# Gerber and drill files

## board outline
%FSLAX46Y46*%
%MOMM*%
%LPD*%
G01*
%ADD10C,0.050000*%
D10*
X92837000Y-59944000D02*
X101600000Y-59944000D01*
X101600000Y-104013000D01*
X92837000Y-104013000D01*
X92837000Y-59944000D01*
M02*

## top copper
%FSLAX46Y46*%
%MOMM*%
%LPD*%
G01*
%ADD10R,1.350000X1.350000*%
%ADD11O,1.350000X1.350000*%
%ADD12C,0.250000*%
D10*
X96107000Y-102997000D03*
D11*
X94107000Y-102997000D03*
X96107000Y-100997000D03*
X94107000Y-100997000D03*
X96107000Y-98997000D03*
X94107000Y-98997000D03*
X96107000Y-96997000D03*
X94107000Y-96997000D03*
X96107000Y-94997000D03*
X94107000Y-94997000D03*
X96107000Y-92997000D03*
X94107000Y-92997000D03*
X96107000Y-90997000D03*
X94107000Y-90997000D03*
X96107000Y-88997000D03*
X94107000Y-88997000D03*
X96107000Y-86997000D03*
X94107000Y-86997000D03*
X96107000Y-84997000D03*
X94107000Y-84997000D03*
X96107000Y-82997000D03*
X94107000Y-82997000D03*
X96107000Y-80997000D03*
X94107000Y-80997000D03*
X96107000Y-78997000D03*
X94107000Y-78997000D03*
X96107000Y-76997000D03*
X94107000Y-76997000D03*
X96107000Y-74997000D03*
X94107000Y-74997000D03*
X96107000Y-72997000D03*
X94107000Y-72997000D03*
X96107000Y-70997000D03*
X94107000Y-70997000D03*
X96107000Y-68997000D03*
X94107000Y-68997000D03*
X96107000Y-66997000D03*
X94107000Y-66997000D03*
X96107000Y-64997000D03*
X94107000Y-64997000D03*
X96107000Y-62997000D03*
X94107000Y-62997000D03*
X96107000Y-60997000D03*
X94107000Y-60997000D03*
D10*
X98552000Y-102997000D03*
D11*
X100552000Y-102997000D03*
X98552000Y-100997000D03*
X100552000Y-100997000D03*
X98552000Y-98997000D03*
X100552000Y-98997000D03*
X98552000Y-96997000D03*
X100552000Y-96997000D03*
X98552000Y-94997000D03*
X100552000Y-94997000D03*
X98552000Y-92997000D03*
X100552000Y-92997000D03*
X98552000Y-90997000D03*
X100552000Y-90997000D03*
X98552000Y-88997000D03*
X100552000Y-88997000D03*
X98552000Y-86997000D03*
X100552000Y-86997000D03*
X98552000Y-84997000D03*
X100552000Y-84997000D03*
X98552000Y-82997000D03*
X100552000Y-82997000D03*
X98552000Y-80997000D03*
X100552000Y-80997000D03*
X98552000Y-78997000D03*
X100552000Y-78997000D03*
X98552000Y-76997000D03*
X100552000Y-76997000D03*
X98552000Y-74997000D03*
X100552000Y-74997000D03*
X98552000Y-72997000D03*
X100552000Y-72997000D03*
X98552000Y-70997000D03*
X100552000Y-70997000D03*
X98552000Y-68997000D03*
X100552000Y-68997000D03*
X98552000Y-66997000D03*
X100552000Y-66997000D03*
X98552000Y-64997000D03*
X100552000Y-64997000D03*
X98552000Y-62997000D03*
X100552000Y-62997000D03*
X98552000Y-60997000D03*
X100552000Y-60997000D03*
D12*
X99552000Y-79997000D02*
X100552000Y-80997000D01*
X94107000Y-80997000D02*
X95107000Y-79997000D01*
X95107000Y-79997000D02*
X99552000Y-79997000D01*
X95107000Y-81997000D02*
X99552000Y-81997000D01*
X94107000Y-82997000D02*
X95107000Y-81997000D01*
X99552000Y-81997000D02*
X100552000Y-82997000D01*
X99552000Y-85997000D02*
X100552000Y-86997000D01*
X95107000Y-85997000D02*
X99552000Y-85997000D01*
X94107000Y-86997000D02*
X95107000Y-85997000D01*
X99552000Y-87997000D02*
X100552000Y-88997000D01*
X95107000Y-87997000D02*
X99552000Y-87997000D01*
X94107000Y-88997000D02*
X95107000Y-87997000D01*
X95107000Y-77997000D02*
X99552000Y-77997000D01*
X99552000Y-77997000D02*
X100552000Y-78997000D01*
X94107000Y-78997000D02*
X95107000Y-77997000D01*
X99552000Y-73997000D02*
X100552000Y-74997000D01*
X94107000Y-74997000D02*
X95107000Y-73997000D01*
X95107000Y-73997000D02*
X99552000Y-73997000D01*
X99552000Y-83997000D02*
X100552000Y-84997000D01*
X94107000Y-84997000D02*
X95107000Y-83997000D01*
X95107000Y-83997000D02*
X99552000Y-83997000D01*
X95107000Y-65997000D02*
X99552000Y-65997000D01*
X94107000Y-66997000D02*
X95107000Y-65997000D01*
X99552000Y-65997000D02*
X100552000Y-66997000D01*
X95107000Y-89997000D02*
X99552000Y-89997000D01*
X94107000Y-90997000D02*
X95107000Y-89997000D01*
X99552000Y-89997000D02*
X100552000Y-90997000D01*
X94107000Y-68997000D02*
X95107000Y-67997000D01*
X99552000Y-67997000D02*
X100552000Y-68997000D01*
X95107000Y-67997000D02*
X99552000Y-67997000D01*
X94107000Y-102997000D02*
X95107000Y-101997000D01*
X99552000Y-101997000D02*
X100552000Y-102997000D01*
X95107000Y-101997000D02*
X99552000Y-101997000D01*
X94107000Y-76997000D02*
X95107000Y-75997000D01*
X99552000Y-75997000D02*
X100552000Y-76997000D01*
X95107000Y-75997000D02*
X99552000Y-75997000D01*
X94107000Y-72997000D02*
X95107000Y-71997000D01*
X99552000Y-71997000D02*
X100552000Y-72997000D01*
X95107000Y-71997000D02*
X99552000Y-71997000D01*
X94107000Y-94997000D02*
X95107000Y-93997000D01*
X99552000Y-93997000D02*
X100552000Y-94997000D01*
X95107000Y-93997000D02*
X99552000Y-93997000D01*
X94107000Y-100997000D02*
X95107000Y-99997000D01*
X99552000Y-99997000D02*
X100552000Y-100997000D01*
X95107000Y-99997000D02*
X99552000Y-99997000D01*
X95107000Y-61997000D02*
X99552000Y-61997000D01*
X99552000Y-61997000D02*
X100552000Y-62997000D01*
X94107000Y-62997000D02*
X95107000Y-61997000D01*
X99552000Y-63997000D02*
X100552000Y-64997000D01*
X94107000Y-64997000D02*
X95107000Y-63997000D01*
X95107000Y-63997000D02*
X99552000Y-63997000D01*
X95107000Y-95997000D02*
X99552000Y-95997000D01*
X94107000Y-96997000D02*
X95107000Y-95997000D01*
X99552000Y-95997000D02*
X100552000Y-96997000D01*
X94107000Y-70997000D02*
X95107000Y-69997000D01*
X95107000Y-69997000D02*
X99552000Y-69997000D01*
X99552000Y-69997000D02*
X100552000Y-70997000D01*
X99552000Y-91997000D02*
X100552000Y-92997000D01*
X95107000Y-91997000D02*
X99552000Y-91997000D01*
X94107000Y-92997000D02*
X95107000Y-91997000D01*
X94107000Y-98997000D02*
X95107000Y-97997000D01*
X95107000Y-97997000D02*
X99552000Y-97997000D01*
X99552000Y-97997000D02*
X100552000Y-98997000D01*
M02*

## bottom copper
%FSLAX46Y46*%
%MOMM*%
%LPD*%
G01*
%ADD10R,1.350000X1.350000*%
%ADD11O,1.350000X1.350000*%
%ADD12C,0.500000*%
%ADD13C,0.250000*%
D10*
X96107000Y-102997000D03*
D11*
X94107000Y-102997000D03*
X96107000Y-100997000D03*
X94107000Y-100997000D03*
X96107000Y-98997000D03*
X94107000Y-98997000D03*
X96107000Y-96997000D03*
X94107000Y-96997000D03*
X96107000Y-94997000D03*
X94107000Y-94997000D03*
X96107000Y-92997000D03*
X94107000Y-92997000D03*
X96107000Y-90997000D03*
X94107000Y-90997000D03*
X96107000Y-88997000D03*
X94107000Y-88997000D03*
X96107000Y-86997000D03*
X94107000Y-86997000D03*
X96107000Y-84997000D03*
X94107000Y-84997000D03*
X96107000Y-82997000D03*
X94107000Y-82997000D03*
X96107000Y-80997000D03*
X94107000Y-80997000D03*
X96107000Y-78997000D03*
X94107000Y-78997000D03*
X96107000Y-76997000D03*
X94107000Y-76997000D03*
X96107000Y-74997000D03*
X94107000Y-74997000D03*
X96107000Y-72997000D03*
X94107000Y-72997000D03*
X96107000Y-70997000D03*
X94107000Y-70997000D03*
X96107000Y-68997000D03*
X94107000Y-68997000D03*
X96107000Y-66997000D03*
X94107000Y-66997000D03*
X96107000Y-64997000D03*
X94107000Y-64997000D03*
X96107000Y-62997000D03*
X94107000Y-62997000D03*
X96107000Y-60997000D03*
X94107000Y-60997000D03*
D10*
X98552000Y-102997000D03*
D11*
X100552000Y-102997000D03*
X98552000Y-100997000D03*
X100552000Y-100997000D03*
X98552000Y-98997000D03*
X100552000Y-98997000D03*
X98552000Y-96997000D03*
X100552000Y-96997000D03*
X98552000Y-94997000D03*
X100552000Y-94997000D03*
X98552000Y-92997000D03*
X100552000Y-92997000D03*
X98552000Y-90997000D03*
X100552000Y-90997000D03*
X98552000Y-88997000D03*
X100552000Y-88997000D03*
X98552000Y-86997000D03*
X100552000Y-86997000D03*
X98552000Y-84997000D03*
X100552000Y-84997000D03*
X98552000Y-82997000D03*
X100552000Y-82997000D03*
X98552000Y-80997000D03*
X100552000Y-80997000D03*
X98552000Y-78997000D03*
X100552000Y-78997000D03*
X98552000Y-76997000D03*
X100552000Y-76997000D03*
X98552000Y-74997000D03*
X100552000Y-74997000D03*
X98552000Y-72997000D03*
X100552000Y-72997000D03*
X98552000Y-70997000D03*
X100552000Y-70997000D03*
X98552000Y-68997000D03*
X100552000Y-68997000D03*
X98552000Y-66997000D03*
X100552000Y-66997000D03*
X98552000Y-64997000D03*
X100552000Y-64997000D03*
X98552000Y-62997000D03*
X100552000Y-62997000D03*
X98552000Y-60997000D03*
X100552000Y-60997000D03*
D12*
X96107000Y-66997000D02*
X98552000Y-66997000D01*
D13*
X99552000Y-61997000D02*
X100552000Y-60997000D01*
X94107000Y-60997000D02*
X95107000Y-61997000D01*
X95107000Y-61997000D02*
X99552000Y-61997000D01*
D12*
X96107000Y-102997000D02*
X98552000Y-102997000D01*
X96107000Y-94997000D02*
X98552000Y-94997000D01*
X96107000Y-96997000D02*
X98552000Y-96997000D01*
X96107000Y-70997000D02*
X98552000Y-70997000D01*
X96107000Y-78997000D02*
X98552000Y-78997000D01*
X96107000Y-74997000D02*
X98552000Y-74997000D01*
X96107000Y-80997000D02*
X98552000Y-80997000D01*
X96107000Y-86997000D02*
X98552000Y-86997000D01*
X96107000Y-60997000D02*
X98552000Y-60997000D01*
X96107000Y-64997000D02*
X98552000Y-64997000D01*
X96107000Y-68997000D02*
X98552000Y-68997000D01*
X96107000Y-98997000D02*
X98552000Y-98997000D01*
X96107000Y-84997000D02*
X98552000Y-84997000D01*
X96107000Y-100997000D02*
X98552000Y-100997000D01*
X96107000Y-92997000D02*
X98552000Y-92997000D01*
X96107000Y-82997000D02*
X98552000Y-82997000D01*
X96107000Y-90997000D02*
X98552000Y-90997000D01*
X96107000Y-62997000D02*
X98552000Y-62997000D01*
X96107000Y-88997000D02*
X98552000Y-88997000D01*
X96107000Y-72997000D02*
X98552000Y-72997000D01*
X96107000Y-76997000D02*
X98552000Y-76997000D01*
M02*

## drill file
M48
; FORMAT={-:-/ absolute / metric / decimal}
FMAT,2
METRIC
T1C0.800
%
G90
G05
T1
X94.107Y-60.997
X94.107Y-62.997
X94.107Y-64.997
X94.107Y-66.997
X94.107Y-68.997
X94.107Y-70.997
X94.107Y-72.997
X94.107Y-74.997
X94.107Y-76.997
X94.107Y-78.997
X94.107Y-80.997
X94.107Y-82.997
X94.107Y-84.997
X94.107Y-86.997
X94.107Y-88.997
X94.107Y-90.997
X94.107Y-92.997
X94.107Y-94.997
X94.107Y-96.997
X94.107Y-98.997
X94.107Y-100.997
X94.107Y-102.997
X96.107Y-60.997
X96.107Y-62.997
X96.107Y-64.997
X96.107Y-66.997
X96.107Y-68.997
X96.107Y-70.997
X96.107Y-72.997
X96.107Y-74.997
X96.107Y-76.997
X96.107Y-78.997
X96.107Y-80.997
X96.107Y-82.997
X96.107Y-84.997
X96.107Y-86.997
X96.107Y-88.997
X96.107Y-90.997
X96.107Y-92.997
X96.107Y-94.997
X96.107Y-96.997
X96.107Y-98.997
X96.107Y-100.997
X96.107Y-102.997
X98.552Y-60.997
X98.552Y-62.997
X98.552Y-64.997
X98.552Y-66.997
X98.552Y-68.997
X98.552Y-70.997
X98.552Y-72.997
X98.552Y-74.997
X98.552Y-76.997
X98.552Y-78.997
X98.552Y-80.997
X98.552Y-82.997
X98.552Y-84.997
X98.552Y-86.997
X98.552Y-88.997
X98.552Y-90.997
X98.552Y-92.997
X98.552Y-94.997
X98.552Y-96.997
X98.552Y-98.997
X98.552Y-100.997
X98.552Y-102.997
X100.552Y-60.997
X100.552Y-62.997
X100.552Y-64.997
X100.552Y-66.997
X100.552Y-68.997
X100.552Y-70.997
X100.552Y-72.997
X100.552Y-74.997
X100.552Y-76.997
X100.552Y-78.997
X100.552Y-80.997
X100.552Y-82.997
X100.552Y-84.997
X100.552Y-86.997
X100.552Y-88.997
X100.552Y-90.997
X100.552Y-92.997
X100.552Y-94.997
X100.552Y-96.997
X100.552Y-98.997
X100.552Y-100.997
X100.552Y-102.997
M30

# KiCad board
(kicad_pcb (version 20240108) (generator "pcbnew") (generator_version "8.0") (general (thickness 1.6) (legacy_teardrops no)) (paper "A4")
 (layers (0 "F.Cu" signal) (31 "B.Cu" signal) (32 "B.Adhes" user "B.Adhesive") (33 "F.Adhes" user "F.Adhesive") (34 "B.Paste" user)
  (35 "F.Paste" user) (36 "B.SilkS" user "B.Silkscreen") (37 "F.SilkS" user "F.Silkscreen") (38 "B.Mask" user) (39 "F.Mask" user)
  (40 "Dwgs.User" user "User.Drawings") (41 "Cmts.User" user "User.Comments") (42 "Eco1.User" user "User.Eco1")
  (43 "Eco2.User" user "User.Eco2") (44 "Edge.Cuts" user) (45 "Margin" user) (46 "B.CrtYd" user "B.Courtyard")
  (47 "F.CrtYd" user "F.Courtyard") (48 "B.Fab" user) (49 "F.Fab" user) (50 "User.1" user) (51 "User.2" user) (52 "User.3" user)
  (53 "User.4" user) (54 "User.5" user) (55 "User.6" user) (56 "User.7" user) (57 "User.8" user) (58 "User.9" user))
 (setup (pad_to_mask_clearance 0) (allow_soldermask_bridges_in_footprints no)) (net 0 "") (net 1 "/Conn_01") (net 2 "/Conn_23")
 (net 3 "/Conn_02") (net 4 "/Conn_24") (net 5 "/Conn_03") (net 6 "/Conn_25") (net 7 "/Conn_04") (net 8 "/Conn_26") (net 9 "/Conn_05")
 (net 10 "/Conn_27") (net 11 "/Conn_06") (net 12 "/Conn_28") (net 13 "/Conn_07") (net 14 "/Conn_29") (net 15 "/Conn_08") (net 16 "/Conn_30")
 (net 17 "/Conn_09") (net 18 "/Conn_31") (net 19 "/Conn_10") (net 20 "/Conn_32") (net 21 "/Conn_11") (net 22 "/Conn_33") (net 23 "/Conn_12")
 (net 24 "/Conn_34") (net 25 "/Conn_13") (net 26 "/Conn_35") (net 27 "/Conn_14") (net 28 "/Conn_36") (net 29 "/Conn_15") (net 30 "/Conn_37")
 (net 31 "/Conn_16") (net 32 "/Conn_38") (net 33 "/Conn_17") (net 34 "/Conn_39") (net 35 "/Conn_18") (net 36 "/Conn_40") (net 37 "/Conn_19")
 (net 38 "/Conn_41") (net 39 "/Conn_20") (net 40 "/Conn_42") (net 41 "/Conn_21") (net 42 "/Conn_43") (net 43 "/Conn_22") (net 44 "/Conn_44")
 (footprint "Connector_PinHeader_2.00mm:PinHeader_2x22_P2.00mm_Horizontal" (layer "F.Cu") (at 96.107 102.997 180)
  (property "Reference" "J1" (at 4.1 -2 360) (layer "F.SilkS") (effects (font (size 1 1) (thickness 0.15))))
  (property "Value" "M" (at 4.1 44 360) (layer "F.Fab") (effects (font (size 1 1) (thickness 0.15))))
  (pad "1" thru_hole rect (at 0 0 180) (size 1.35 1.35) (drill 0.8) (layers "*.Cu" "*.Mask") (remove_unused_layers no) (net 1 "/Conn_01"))
  (pad "2" thru_hole oval (at 2 0 180) (size 1.35 1.35) (drill 0.8) (layers "*.Cu" "*.Mask") (remove_unused_layers no) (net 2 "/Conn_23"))
  (pad "3" thru_hole oval (at 0 2 180) (size 1.35 1.35) (drill 0.8) (layers "*.Cu" "*.Mask") (remove_unused_layers no) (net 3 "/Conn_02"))
  (pad "4" thru_hole oval (at 2 2 180) (size 1.35 1.35) (drill 0.8) (layers "*.Cu" "*.Mask") (remove_unused_layers no) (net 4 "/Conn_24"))
  (pad "5" thru_hole oval (at 0 4 180) (size 1.35 1.35) (drill 0.8) (layers "*.Cu" "*.Mask") (remove_unused_layers no) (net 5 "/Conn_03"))
  (pad "6" thru_hole oval (at 2 4 180) (size 1.35 1.35) (drill 0.8) (layers "*.Cu" "*.Mask") (remove_unused_layers no) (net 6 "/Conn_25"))
  (pad "7" thru_hole oval (at 0 6 180) (size 1.35 1.35) (drill 0.8) (layers "*.Cu" "*.Mask") (remove_unused_layers no) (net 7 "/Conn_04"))
  (pad "8" thru_hole oval (at 2 6 180) (size 1.35 1.35) (drill 0.8) (layers "*.Cu" "*.Mask") (remove_unused_layers no) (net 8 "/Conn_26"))
  (pad "9" thru_hole oval (at 0 8 180) (size 1.35 1.35) (drill 0.8) (layers "*.Cu" "*.Mask") (remove_unused_layers no) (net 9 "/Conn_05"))
  (pad "10" thru_hole oval (at 2 8 180) (size 1.35 1.35) (drill 0.8) (layers "*.Cu" "*.Mask") (remove_unused_layers no) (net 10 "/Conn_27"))
  (pad "11" thru_hole oval (at 0 10 180) (size 1.35 1.35) (drill 0.8) (layers "*.Cu" "*.Mask") (remove_unused_layers no) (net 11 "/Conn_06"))
  (pad "12" thru_hole oval (at 2 10 180) (size 1.35 1.35) (drill 0.8) (layers "*.Cu" "*.Mask") (remove_unused_layers no) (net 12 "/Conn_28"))
  (pad "13" thru_hole oval (at 0 12 180) (size 1.35 1.35) (drill 0.8) (layers "*.Cu" "*.Mask") (remove_unused_layers no) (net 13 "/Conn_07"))
  (pad "14" thru_hole oval (at 2 12 180) (size 1.35 1.35) (drill 0.8) (layers "*.Cu" "*.Mask") (remove_unused_layers no) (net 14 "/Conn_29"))
  (pad "15" thru_hole oval (at 0 14 180) (size 1.35 1.35) (drill 0.8) (layers "*.Cu" "*.Mask") (remove_unused_layers no) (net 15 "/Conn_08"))
  (pad "16" thru_hole oval (at 2 14 180) (size 1.35 1.35) (drill 0.8) (layers "*.Cu" "*.Mask") (remove_unused_layers no) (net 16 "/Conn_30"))
  (pad "17" thru_hole oval (at 0 16 180) (size 1.35 1.35) (drill 0.8) (layers "*.Cu" "*.Mask") (remove_unused_layers no) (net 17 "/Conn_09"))
  (pad "18" thru_hole oval (at 2 16 180) (size 1.35 1.35) (drill 0.8) (layers "*.Cu" "*.Mask") (remove_unused_layers no) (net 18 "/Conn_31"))
  (pad "19" thru_hole oval (at 0 18 180) (size 1.35 1.35) (drill 0.8) (layers "*.Cu" "*.Mask") (remove_unused_layers no) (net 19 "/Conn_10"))
  (pad "20" thru_hole oval (at 2 18 180) (size 1.35 1.35) (drill 0.8) (layers "*.Cu" "*.Mask") (remove_unused_layers no) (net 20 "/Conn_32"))
  (pad "21" thru_hole oval (at 0 20 180) (size 1.35 1.35) (drill 0.8) (layers "*.Cu" "*.Mask") (remove_unused_layers no) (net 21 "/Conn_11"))
  (pad "22" thru_hole oval (at 2 20 180) (size 1.35 1.35) (drill 0.8) (layers "*.Cu" "*.Mask") (remove_unused_layers no) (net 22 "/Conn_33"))
  (pad "23" thru_hole oval (at 0 22 180) (size 1.35 1.35) (drill 0.8) (layers "*.Cu" "*.Mask") (remove_unused_layers no) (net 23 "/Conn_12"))
  (pad "24" thru_hole oval (at 2 22 180) (size 1.35 1.35) (drill 0.8) (layers "*.Cu" "*.Mask") (remove_unused_layers no) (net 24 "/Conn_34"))
  (pad "25" thru_hole oval (at 0 24 180) (size 1.35 1.35) (drill 0.8) (layers "*.Cu" "*.Mask") (remove_unused_layers no) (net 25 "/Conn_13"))
  (pad "26" thru_hole oval (at 2 24 180) (size 1.35 1.35) (drill 0.8) (layers "*.Cu" "*.Mask") (remove_unused_layers no) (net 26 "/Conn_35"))
  (pad "27" thru_hole oval (at 0 26 180) (size 1.35 1.35) (drill 0.8) (layers "*.Cu" "*.Mask") (remove_unused_layers no) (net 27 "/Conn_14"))
  (pad "28" thru_hole oval (at 2 26 180) (size 1.35 1.35) (drill 0.8) (layers "*.Cu" "*.Mask") (remove_unused_layers no) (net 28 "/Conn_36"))
  (pad "29" thru_hole oval (at 0 28 180) (size 1.35 1.35) (drill 0.8) (layers "*.Cu" "*.Mask") (remove_unused_layers no) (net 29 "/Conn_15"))
  (pad "30" thru_hole oval (at 2 28 180) (size 1.35 1.35) (drill 0.8) (layers "*.Cu" "*.Mask") (remove_unused_layers no) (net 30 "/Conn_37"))
  (pad "31" thru_hole oval (at 0 30 180) (size 1.35 1.35) (drill 0.8) (layers "*.Cu" "*.Mask") (remove_unused_layers no) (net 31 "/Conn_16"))
  (pad "32" thru_hole oval (at 2 30 180) (size 1.35 1.35) (drill 0.8) (layers "*.Cu" "*.Mask") (remove_unused_layers no) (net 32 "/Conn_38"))
  (pad "33" thru_hole oval (at 0 32 180) (size 1.35 1.35) (drill 0.8) (layers "*.Cu" "*.Mask") (remove_unused_layers no) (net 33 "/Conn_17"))
  (pad "34" thru_hole oval (at 2 32 180) (size 1.35 1.35) (drill 0.8) (layers "*.Cu" "*.Mask") (remove_unused_layers no) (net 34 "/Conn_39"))
  (pad "35" thru_hole oval (at 0 34 180) (size 1.35 1.35) (drill 0.8) (layers "*.Cu" "*.Mask") (remove_unused_layers no) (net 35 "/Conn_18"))
  (pad "36" thru_hole oval (at 2 34 180) (size 1.35 1.35) (drill 0.8) (layers "*.Cu" "*.Mask") (remove_unused_layers no) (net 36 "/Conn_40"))
  (pad "37" thru_hole oval (at 0 36 180) (size 1.35 1.35) (drill 0.8) (layers "*.Cu" "*.Mask") (remove_unused_layers no) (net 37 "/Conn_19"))
  (pad "38" thru_hole oval (at 2 36 180) (size 1.35 1.35) (drill 0.8) (layers "*.Cu" "*.Mask") (remove_unused_layers no) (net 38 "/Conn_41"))
  (pad "39" thru_hole oval (at 0 38 180) (size 1.35 1.35) (drill 0.8) (layers "*.Cu" "*.Mask") (remove_unused_layers no) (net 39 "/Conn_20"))
  (pad "40" thru_hole oval (at 2 38 180) (size 1.35 1.35) (drill 0.8) (layers "*.Cu" "*.Mask") (remove_unused_layers no) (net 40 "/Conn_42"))
  (pad "41" thru_hole oval (at 0 40 180) (size 1.35 1.35) (drill 0.8) (layers "*.Cu" "*.Mask") (remove_unused_layers no) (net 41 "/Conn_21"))
  (pad "42" thru_hole oval (at 2 40 180) (size 1.35 1.35) (drill 0.8) (layers "*.Cu" "*.Mask") (remove_unused_layers no) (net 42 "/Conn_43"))
  (pad "43" thru_hole oval (at 0 42 180) (size 1.35 1.35) (drill 0.8) (layers "*.Cu" "*.Mask") (remove_unused_layers no) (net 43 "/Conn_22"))
  (pad "44" thru_hole oval (at 2 42 180) (size 1.35 1.35) (drill 0.8) (layers "*.Cu" "*.Mask") (remove_unused_layers no) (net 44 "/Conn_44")))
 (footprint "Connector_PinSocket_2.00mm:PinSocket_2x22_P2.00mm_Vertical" (layer "F.Cu") (at 98.552 102.997 180)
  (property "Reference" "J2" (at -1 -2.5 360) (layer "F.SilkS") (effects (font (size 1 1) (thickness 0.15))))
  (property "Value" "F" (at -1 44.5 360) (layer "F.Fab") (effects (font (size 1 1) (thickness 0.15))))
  (pad "1" thru_hole rect (at 0 0 180) (size 1.35 1.35) (drill 0.8) (layers "*.Cu" "*.Mask") (remove_unused_layers no) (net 1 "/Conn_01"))
  (pad "2" thru_hole oval (at -2 0 180) (size 1.35 1.35) (drill 0.8) (layers "*.Cu" "*.Mask") (remove_unused_layers no) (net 2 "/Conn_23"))
  (pad "3" thru_hole oval (at 0 2 180) (size 1.35 1.35) (drill 0.8) (layers "*.Cu" "*.Mask") (remove_unused_layers no) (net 3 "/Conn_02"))
  (pad "4" thru_hole oval (at -2 2 180) (size 1.35 1.35) (drill 0.8) (layers "*.Cu" "*.Mask") (remove_unused_layers no) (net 4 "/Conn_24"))
  (pad "5" thru_hole oval (at 0 4 180) (size 1.35 1.35) (drill 0.8) (layers "*.Cu" "*.Mask") (remove_unused_layers no) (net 5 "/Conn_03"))
  (pad "6" thru_hole oval (at -2 4 180) (size 1.35 1.35) (drill 0.8) (layers "*.Cu" "*.Mask") (remove_unused_layers no) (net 6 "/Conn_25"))
  (pad "7" thru_hole oval (at 0 6 180) (size 1.35 1.35) (drill 0.8) (layers "*.Cu" "*.Mask") (remove_unused_layers no) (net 7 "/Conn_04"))
  (pad "8" thru_hole oval (at -2 6 180) (size 1.35 1.35) (drill 0.8) (layers "*.Cu" "*.Mask") (remove_unused_layers no) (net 8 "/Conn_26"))
  (pad "9" thru_hole oval (at 0 8 180) (size 1.35 1.35) (drill 0.8) (layers "*.Cu" "*.Mask") (remove_unused_layers no) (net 9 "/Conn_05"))
  (pad "10" thru_hole oval (at -2 8 180) (size 1.35 1.35) (drill 0.8) (layers "*.Cu" "*.Mask") (remove_unused_layers no) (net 10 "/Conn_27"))
  (pad "11" thru_hole oval (at 0 10 180) (size 1.35 1.35) (drill 0.8) (layers "*.Cu" "*.Mask") (remove_unused_layers no) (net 11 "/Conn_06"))
  (pad "12" thru_hole oval (at -2 10 180) (size 1.35 1.35) (drill 0.8) (layers "*.Cu" "*.Mask") (remove_unused_layers no)
   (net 12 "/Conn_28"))
  (pad "13" thru_hole oval (at 0 12 180) (size 1.35 1.35) (drill 0.8) (layers "*.Cu" "*.Mask") (remove_unused_layers no) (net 13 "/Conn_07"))
  (pad "14" thru_hole oval (at -2 12 180) (size 1.35 1.35) (drill 0.8) (layers "*.Cu" "*.Mask") (remove_unused_layers no)
   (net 14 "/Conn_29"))
  (pad "15" thru_hole oval (at 0 14 180) (size 1.35 1.35) (drill 0.8) (layers "*.Cu" "*.Mask") (remove_unused_layers no) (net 15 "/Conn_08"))
  (pad "16" thru_hole oval (at -2 14 180) (size 1.35 1.35) (drill 0.8) (layers "*.Cu" "*.Mask") (remove_unused_layers no)
   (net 16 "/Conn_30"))
  (pad "17" thru_hole oval (at 0 16 180) (size 1.35 1.35) (drill 0.8) (layers "*.Cu" "*.Mask") (remove_unused_layers no) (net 17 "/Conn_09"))
  (pad "18" thru_hole oval (at -2 16 180) (size 1.35 1.35) (drill 0.8) (layers "*.Cu" "*.Mask") (remove_unused_layers no)
   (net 18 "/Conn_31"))
  (pad "19" thru_hole oval (at 0 18 180) (size 1.35 1.35) (drill 0.8) (layers "*.Cu" "*.Mask") (remove_unused_layers no) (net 19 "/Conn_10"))
  (pad "20" thru_hole oval (at -2 18 180) (size 1.35 1.35) (drill 0.8) (layers "*.Cu" "*.Mask") (remove_unused_layers no)
   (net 20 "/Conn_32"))
  (pad "21" thru_hole oval (at 0 20 180) (size 1.35 1.35) (drill 0.8) (layers "*.Cu" "*.Mask") (remove_unused_layers no) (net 21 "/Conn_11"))
  (pad "22" thru_hole oval (at -2 20 180) (size 1.35 1.35) (drill 0.8) (layers "*.Cu" "*.Mask") (remove_unused_layers no)
   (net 22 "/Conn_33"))
  (pad "23" thru_hole oval (at 0 22 180) (size 1.35 1.35) (drill 0.8) (layers "*.Cu" "*.Mask") (remove_unused_layers no) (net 23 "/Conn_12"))
  (pad "24" thru_hole oval (at -2 22 180) (size 1.35 1.35) (drill 0.8) (layers "*.Cu" "*.Mask") (remove_unused_layers no)
   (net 24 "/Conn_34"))
  (pad "25" thru_hole oval (at 0 24 180) (size 1.35 1.35) (drill 0.8) (layers "*.Cu" "*.Mask") (remove_unused_layers no) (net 25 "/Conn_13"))
  (pad "26" thru_hole oval (at -2 24 180) (size 1.35 1.35) (drill 0.8) (layers "*.Cu" "*.Mask") (remove_unused_layers no)
   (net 26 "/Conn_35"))
  (pad "27" thru_hole oval (at 0 26 180) (size 1.35 1.35) (drill 0.8) (layers "*.Cu" "*.Mask") (remove_unused_layers no) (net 27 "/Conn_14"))
  (pad "28" thru_hole oval (at -2 26 180) (size 1.35 1.35) (drill 0.8) (layers "*.Cu" "*.Mask") (remove_unused_layers no)
   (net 28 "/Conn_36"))
  (pad "29" thru_hole oval (at 0 28 180) (size 1.35 1.35) (drill 0.8) (layers "*.Cu" "*.Mask") (remove_unused_layers no) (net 29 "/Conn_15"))
  (pad "30" thru_hole oval (at -2 28 180) (size 1.35 1.35) (drill 0.8) (layers "*.Cu" "*.Mask") (remove_unused_layers no)
   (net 30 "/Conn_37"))
  (pad "31" thru_hole oval (at 0 30 180) (size 1.35 1.35) (drill 0.8) (layers "*.Cu" "*.Mask") (remove_unused_layers no) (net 31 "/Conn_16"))
  (pad "32" thru_hole oval (at -2 30 180) (size 1.35 1.35) (drill 0.8) (layers "*.Cu" "*.Mask") (remove_unused_layers no)
   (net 32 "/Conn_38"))
  (pad "33" thru_hole oval (at 0 32 180) (size 1.35 1.35) (drill 0.8) (layers "*.Cu" "*.Mask") (remove_unused_layers no) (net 33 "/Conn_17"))
  (pad "34" thru_hole oval (at -2 32 180) (size 1.35 1.35) (drill 0.8) (layers "*.Cu" "*.Mask") (remove_unused_layers no)
   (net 34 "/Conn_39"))
  (pad "35" thru_hole oval (at 0 34 180) (size 1.35 1.35) (drill 0.8) (layers "*.Cu" "*.Mask") (remove_unused_layers no) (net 35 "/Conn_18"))
  (pad "36" thru_hole oval (at -2 34 180) (size 1.35 1.35) (drill 0.8) (layers "*.Cu" "*.Mask") (remove_unused_layers no)
   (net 36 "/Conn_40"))
  (pad "37" thru_hole oval (at 0 36 180) (size 1.35 1.35) (drill 0.8) (layers "*.Cu" "*.Mask") (remove_unused_layers no) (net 37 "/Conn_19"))
  (pad "38" thru_hole oval (at -2 36 180) (size 1.35 1.35) (drill 0.8) (layers "*.Cu" "*.Mask") (remove_unused_layers no)
   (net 38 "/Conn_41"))
  (pad "39" thru_hole oval (at 0 38 180) (size 1.35 1.35) (drill 0.8) (layers "*.Cu" "*.Mask") (remove_unused_layers no) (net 39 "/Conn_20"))
  (pad "40" thru_hole oval (at -2 38 180) (size 1.35 1.35) (drill 0.8) (layers "*.Cu" "*.Mask") (remove_unused_layers no)
   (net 40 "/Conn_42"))
  (pad "41" thru_hole oval (at 0 40 180) (size 1.35 1.35) (drill 0.8) (layers "*.Cu" "*.Mask") (remove_unused_layers no) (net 41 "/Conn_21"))
  (pad "42" thru_hole oval (at -2 40 180) (size 1.35 1.35) (drill 0.8) (layers "*.Cu" "*.Mask") (remove_unused_layers no)
   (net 42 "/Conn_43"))
  (pad "43" thru_hole oval (at 0 42 180) (size 1.35 1.35) (drill 0.8) (layers "*.Cu" "*.Mask") (remove_unused_layers no) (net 43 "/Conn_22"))
  (pad "44" thru_hole oval (at -2 42 180) (size 1.35 1.35) (drill 0.8) (layers "*.Cu" "*.Mask") (remove_unused_layers no)
   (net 44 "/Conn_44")))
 (gr_rect (start 92.837 59.944) (end 101.6 104.013) (stroke (width 0.05) (type default)) (fill none) (layer "Edge.Cuts"))
 (segment (start 99.552 79.997) (end 100.552 80.997) (width 0.25) (layer "F.Cu") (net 24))
 (segment (start 94.107 80.997) (end 95.107 79.997) (width 0.25) (layer "F.Cu") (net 24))
 (segment (start 95.107 79.997) (end 99.552 79.997) (width 0.25) (layer "F.Cu") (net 24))
 (segment (start 96.107 66.997) (end 98.552 66.997) (width 0.5) (layer "B.Cu") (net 37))
 (segment (start 95.107 81.997) (end 99.552 81.997) (width 0.25) (layer "F.Cu") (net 22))
 (segment (start 94.107 82.997) (end 95.107 81.997) (width 0.25) (layer "F.Cu") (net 22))
 (segment (start 99.552 81.997) (end 100.552 82.997) (width 0.25) (layer "F.Cu") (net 22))
 (segment (start 99.552 85.997) (end 100.552 86.997) (width 0.25) (layer "F.Cu") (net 18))
 (segment (start 95.107 85.997) (end 99.552 85.997) (width 0.25) (layer "F.Cu") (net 18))
 (segment (start 94.107 86.997) (end 95.107 85.997) (width 0.25) (layer "F.Cu") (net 18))
 (segment (start 99.552 61.997) (end 100.552 60.997) (width 0.25) (layer "B.Cu") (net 44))
 (segment (start 94.107 60.997) (end 95.107 61.997) (width 0.25) (layer "B.Cu") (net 44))
 (segment (start 95.107 61.997) (end 99.552 61.997) (width 0.25) (layer "B.Cu") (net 44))
 (segment (start 99.552 87.997) (end 100.552 88.997) (width 0.25) (layer "F.Cu") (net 16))
 (segment (start 95.107 87.997) (end 99.552 87.997) (width 0.25) (layer "F.Cu") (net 16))
 (segment (start 94.107 88.997) (end 95.107 87.997) (width 0.25) (layer "F.Cu") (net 16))
 (segment (start 95.107 77.997) (end 99.552 77.997) (width 0.25) (layer "F.Cu") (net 26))
 (segment (start 99.552 77.997) (end 100.552 78.997) (width 0.25) (layer "F.Cu") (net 26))
 (segment (start 94.107 78.997) (end 95.107 77.997) (width 0.25) (layer "F.Cu") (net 26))
 (segment (start 96.107 102.997) (end 98.552 102.997) (width 0.5) (layer "B.Cu") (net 1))
 (segment (start 96.107 94.997) (end 98.552 94.997) (width 0.5) (layer "B.Cu") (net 9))
 (segment (start 96.107 96.997) (end 98.552 96.997) (width 0.5) (layer "B.Cu") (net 7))
 (segment (start 99.552 73.997) (end 100.552 74.997) (width 0.25) (layer "F.Cu") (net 30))
 (segment (start 94.107 74.997) (end 95.107 73.997) (width 0.25) (layer "F.Cu") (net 30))
 (segment (start 95.107 73.997) (end 99.552 73.997) (width 0.25) (layer "F.Cu") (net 30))
 (segment (start 96.107 70.997) (end 98.552 70.997) (width 0.5) (layer "B.Cu") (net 33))
 (segment (start 96.107 78.997) (end 98.552 78.997) (width 0.5) (layer "B.Cu") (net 25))
 (segment (start 99.552 83.997) (end 100.552 84.997) (width 0.25) (layer "F.Cu") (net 20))
 (segment (start 94.107 84.997) (end 95.107 83.997) (width 0.25) (layer "F.Cu") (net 20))
 (segment (start 95.107 83.997) (end 99.552 83.997) (width 0.25) (layer "F.Cu") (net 20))
 (segment (start 96.107 74.997) (end 98.552 74.997) (width 0.5) (layer "B.Cu") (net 29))
 (segment (start 96.107 80.997) (end 98.552 80.997) (width 0.5) (layer "B.Cu") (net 23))
 (segment (start 96.107 86.997) (end 98.552 86.997) (width 0.5) (layer "B.Cu") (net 17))
 (segment (start 96.107 60.997) (end 98.552 60.997) (width 0.5) (layer "B.Cu") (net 43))
 (segment (start 95.107 65.997) (end 99.552 65.997) (width 0.25) (layer "F.Cu") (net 38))
 (segment (start 94.107 66.997) (end 95.107 65.997) (width 0.25) (layer "F.Cu") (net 38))
 (segment (start 99.552 65.997) (end 100.552 66.997) (width 0.25) (layer "F.Cu") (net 38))
 (segment (start 96.107 64.997) (end 98.552 64.997) (width 0.5) (layer "B.Cu") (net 39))
 (segment (start 95.107 89.997) (end 99.552 89.997) (width 0.25) (layer "F.Cu") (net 14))
 (segment (start 94.107 90.997) (end 95.107 89.997) (width 0.25) (layer "F.Cu") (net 14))
 (segment (start 99.552 89.997) (end 100.552 90.997) (width 0.25) (layer "F.Cu") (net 14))
 (segment (start 94.107 68.997) (end 95.107 67.997) (width 0.25) (layer "F.Cu") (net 36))
 (segment (start 99.552 67.997) (end 100.552 68.997) (width 0.25) (layer "F.Cu") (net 36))
 (segment (start 95.107 67.997) (end 99.552 67.997) (width 0.25) (layer "F.Cu") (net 36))
 (segment (start 94.107 102.997) (end 95.107 101.997) (width 0.25) (layer "F.Cu") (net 2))
 (segment (start 99.552 101.997) (end 100.552 102.997) (width 0.25) (layer "F.Cu") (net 2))
 (segment (start 95.107 101.997) (end 99.552 101.997) (width 0.25) (layer "F.Cu") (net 2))
 (segment (start 96.107 68.997) (end 98.552 68.997) (width 0.5) (layer "B.Cu") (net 35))
 (segment (start 96.107 98.997) (end 98.552 98.997) (width 0.5) (layer "B.Cu") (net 5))
 (segment (start 94.107 76.997) (end 95.107 75.997) (width 0.25) (layer "F.Cu") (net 28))
 (segment (start 99.552 75.997) (end 100.552 76.997) (width 0.25) (layer "F.Cu") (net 28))
 (segment (start 95.107 75.997) (end 99.552 75.997) (width 0.25) (layer "F.Cu") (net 28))
 (segment (start 96.107 84.997) (end 98.552 84.997) (width 0.5) (layer "B.Cu") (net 19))
 (segment (start 94.107 72.997) (end 95.107 71.997) (width 0.25) (layer "F.Cu") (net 32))
 (segment (start 99.552 71.997) (end 100.552 72.997) (width 0.25) (layer "F.Cu") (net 32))
 (segment (start 95.107 71.997) (end 99.552 71.997) (width 0.25) (layer "F.Cu") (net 32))
 (segment (start 94.107 94.997) (end 95.107 93.997) (width 0.25) (layer "F.Cu") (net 10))
 (segment (start 99.552 93.997) (end 100.552 94.997) (width 0.25) (layer "F.Cu") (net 10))
 (segment (start 95.107 93.997) (end 99.552 93.997) (width 0.25) (layer "F.Cu") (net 10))
 (segment (start 94.107 100.997) (end 95.107 99.997) (width 0.25) (layer "F.Cu") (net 4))
 (segment (start 99.552 99.997) (end 100.552 100.997) (width 0.25) (layer "F.Cu") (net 4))
 (segment (start 95.107 99.997) (end 99.552 99.997) (width 0.25) (layer "F.Cu") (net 4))
 (segment (start 96.107 100.997) (end 98.552 100.997) (width 0.5) (layer "B.Cu") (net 3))
 (segment (start 96.107 92.997) (end 98.552 92.997) (width 0.5) (layer "B.Cu") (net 11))
 (segment (start 96.107 82.997) (end 98.552 82.997) (width 0.5) (layer "B.Cu") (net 21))
 (segment (start 96.107 90.997) (end 98.552 90.997) (width 0.5) (layer "B.Cu") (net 13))
 (segment (start 95.107 61.997) (end 99.552 61.997) (width 0.25) (layer "F.Cu") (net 42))
 (segment (start 99.552 61.997) (end 100.552 62.997) (width 0.25) (layer "F.Cu") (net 42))
 (segment (start 94.107 62.997) (end 95.107 61.997) (width 0.25) (layer "F.Cu") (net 42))
 (segment (start 99.552 63.997) (end 100.552 64.997) (width 0.25) (layer "F.Cu") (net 40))
 (segment (start 94.107 64.997) (end 95.107 63.997) (width 0.25) (layer "F.Cu") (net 40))
 (segment (start 95.107 63.997) (end 99.552 63.997) (width 0.25) (layer "F.Cu") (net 40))
 (segment (start 95.107 95.997) (end 99.552 95.997) (width 0.25) (layer "F.Cu") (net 8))
 (segment (start 94.107 96.997) (end 95.107 95.997) (width 0.25) (layer "F.Cu") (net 8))
 (segment (start 99.552 95.997) (end 100.552 96.997) (width 0.25) (layer "F.Cu") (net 8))
 (segment (start 96.107 62.997) (end 98.552 62.997) (width 0.5) (layer "B.Cu") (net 41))
 (segment (start 94.107 70.997) (end 95.107 69.997) (width 0.25) (layer "F.Cu") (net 34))
 (segment (start 95.107 69.997) (end 99.552 69.997) (width 0.25) (layer "F.Cu") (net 34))
 (segment (start 99.552 69.997) (end 100.552 70.997) (width 0.25) (layer "F.Cu") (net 34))
 (segment (start 99.552 91.997) (end 100.552 92.997) (width 0.25) (layer "F.Cu") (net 12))
 (segment (start 95.107 91.997) (end 99.552 91.997) (width 0.25) (layer "F.Cu") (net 12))
 (segment (start 94.107 92.997) (end 95.107 91.997) (width 0.25) (layer "F.Cu") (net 12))
 (segment (start 96.107 88.997) (end 98.552 88.997) (width 0.5) (layer "B.Cu") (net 15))
 (segment (start 94.107 98.997) (end 95.107 97.997) (width 0.25) (layer "F.Cu") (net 6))
 (segment (start 95.107 97.997) (end 99.552 97.997) (width 0.25) (layer "F.Cu") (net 6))
 (segment (start 99.552 97.997) (end 100.552 98.997) (width 0.25) (layer "F.Cu") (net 6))
 (segment (start 96.107 72.997) (end 98.552 72.997) (width 0.5) (layer "B.Cu") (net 31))
 (segment (start 96.107 76.997) (end 98.552 76.997) (width 0.5) (layer "B.Cu") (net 27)))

